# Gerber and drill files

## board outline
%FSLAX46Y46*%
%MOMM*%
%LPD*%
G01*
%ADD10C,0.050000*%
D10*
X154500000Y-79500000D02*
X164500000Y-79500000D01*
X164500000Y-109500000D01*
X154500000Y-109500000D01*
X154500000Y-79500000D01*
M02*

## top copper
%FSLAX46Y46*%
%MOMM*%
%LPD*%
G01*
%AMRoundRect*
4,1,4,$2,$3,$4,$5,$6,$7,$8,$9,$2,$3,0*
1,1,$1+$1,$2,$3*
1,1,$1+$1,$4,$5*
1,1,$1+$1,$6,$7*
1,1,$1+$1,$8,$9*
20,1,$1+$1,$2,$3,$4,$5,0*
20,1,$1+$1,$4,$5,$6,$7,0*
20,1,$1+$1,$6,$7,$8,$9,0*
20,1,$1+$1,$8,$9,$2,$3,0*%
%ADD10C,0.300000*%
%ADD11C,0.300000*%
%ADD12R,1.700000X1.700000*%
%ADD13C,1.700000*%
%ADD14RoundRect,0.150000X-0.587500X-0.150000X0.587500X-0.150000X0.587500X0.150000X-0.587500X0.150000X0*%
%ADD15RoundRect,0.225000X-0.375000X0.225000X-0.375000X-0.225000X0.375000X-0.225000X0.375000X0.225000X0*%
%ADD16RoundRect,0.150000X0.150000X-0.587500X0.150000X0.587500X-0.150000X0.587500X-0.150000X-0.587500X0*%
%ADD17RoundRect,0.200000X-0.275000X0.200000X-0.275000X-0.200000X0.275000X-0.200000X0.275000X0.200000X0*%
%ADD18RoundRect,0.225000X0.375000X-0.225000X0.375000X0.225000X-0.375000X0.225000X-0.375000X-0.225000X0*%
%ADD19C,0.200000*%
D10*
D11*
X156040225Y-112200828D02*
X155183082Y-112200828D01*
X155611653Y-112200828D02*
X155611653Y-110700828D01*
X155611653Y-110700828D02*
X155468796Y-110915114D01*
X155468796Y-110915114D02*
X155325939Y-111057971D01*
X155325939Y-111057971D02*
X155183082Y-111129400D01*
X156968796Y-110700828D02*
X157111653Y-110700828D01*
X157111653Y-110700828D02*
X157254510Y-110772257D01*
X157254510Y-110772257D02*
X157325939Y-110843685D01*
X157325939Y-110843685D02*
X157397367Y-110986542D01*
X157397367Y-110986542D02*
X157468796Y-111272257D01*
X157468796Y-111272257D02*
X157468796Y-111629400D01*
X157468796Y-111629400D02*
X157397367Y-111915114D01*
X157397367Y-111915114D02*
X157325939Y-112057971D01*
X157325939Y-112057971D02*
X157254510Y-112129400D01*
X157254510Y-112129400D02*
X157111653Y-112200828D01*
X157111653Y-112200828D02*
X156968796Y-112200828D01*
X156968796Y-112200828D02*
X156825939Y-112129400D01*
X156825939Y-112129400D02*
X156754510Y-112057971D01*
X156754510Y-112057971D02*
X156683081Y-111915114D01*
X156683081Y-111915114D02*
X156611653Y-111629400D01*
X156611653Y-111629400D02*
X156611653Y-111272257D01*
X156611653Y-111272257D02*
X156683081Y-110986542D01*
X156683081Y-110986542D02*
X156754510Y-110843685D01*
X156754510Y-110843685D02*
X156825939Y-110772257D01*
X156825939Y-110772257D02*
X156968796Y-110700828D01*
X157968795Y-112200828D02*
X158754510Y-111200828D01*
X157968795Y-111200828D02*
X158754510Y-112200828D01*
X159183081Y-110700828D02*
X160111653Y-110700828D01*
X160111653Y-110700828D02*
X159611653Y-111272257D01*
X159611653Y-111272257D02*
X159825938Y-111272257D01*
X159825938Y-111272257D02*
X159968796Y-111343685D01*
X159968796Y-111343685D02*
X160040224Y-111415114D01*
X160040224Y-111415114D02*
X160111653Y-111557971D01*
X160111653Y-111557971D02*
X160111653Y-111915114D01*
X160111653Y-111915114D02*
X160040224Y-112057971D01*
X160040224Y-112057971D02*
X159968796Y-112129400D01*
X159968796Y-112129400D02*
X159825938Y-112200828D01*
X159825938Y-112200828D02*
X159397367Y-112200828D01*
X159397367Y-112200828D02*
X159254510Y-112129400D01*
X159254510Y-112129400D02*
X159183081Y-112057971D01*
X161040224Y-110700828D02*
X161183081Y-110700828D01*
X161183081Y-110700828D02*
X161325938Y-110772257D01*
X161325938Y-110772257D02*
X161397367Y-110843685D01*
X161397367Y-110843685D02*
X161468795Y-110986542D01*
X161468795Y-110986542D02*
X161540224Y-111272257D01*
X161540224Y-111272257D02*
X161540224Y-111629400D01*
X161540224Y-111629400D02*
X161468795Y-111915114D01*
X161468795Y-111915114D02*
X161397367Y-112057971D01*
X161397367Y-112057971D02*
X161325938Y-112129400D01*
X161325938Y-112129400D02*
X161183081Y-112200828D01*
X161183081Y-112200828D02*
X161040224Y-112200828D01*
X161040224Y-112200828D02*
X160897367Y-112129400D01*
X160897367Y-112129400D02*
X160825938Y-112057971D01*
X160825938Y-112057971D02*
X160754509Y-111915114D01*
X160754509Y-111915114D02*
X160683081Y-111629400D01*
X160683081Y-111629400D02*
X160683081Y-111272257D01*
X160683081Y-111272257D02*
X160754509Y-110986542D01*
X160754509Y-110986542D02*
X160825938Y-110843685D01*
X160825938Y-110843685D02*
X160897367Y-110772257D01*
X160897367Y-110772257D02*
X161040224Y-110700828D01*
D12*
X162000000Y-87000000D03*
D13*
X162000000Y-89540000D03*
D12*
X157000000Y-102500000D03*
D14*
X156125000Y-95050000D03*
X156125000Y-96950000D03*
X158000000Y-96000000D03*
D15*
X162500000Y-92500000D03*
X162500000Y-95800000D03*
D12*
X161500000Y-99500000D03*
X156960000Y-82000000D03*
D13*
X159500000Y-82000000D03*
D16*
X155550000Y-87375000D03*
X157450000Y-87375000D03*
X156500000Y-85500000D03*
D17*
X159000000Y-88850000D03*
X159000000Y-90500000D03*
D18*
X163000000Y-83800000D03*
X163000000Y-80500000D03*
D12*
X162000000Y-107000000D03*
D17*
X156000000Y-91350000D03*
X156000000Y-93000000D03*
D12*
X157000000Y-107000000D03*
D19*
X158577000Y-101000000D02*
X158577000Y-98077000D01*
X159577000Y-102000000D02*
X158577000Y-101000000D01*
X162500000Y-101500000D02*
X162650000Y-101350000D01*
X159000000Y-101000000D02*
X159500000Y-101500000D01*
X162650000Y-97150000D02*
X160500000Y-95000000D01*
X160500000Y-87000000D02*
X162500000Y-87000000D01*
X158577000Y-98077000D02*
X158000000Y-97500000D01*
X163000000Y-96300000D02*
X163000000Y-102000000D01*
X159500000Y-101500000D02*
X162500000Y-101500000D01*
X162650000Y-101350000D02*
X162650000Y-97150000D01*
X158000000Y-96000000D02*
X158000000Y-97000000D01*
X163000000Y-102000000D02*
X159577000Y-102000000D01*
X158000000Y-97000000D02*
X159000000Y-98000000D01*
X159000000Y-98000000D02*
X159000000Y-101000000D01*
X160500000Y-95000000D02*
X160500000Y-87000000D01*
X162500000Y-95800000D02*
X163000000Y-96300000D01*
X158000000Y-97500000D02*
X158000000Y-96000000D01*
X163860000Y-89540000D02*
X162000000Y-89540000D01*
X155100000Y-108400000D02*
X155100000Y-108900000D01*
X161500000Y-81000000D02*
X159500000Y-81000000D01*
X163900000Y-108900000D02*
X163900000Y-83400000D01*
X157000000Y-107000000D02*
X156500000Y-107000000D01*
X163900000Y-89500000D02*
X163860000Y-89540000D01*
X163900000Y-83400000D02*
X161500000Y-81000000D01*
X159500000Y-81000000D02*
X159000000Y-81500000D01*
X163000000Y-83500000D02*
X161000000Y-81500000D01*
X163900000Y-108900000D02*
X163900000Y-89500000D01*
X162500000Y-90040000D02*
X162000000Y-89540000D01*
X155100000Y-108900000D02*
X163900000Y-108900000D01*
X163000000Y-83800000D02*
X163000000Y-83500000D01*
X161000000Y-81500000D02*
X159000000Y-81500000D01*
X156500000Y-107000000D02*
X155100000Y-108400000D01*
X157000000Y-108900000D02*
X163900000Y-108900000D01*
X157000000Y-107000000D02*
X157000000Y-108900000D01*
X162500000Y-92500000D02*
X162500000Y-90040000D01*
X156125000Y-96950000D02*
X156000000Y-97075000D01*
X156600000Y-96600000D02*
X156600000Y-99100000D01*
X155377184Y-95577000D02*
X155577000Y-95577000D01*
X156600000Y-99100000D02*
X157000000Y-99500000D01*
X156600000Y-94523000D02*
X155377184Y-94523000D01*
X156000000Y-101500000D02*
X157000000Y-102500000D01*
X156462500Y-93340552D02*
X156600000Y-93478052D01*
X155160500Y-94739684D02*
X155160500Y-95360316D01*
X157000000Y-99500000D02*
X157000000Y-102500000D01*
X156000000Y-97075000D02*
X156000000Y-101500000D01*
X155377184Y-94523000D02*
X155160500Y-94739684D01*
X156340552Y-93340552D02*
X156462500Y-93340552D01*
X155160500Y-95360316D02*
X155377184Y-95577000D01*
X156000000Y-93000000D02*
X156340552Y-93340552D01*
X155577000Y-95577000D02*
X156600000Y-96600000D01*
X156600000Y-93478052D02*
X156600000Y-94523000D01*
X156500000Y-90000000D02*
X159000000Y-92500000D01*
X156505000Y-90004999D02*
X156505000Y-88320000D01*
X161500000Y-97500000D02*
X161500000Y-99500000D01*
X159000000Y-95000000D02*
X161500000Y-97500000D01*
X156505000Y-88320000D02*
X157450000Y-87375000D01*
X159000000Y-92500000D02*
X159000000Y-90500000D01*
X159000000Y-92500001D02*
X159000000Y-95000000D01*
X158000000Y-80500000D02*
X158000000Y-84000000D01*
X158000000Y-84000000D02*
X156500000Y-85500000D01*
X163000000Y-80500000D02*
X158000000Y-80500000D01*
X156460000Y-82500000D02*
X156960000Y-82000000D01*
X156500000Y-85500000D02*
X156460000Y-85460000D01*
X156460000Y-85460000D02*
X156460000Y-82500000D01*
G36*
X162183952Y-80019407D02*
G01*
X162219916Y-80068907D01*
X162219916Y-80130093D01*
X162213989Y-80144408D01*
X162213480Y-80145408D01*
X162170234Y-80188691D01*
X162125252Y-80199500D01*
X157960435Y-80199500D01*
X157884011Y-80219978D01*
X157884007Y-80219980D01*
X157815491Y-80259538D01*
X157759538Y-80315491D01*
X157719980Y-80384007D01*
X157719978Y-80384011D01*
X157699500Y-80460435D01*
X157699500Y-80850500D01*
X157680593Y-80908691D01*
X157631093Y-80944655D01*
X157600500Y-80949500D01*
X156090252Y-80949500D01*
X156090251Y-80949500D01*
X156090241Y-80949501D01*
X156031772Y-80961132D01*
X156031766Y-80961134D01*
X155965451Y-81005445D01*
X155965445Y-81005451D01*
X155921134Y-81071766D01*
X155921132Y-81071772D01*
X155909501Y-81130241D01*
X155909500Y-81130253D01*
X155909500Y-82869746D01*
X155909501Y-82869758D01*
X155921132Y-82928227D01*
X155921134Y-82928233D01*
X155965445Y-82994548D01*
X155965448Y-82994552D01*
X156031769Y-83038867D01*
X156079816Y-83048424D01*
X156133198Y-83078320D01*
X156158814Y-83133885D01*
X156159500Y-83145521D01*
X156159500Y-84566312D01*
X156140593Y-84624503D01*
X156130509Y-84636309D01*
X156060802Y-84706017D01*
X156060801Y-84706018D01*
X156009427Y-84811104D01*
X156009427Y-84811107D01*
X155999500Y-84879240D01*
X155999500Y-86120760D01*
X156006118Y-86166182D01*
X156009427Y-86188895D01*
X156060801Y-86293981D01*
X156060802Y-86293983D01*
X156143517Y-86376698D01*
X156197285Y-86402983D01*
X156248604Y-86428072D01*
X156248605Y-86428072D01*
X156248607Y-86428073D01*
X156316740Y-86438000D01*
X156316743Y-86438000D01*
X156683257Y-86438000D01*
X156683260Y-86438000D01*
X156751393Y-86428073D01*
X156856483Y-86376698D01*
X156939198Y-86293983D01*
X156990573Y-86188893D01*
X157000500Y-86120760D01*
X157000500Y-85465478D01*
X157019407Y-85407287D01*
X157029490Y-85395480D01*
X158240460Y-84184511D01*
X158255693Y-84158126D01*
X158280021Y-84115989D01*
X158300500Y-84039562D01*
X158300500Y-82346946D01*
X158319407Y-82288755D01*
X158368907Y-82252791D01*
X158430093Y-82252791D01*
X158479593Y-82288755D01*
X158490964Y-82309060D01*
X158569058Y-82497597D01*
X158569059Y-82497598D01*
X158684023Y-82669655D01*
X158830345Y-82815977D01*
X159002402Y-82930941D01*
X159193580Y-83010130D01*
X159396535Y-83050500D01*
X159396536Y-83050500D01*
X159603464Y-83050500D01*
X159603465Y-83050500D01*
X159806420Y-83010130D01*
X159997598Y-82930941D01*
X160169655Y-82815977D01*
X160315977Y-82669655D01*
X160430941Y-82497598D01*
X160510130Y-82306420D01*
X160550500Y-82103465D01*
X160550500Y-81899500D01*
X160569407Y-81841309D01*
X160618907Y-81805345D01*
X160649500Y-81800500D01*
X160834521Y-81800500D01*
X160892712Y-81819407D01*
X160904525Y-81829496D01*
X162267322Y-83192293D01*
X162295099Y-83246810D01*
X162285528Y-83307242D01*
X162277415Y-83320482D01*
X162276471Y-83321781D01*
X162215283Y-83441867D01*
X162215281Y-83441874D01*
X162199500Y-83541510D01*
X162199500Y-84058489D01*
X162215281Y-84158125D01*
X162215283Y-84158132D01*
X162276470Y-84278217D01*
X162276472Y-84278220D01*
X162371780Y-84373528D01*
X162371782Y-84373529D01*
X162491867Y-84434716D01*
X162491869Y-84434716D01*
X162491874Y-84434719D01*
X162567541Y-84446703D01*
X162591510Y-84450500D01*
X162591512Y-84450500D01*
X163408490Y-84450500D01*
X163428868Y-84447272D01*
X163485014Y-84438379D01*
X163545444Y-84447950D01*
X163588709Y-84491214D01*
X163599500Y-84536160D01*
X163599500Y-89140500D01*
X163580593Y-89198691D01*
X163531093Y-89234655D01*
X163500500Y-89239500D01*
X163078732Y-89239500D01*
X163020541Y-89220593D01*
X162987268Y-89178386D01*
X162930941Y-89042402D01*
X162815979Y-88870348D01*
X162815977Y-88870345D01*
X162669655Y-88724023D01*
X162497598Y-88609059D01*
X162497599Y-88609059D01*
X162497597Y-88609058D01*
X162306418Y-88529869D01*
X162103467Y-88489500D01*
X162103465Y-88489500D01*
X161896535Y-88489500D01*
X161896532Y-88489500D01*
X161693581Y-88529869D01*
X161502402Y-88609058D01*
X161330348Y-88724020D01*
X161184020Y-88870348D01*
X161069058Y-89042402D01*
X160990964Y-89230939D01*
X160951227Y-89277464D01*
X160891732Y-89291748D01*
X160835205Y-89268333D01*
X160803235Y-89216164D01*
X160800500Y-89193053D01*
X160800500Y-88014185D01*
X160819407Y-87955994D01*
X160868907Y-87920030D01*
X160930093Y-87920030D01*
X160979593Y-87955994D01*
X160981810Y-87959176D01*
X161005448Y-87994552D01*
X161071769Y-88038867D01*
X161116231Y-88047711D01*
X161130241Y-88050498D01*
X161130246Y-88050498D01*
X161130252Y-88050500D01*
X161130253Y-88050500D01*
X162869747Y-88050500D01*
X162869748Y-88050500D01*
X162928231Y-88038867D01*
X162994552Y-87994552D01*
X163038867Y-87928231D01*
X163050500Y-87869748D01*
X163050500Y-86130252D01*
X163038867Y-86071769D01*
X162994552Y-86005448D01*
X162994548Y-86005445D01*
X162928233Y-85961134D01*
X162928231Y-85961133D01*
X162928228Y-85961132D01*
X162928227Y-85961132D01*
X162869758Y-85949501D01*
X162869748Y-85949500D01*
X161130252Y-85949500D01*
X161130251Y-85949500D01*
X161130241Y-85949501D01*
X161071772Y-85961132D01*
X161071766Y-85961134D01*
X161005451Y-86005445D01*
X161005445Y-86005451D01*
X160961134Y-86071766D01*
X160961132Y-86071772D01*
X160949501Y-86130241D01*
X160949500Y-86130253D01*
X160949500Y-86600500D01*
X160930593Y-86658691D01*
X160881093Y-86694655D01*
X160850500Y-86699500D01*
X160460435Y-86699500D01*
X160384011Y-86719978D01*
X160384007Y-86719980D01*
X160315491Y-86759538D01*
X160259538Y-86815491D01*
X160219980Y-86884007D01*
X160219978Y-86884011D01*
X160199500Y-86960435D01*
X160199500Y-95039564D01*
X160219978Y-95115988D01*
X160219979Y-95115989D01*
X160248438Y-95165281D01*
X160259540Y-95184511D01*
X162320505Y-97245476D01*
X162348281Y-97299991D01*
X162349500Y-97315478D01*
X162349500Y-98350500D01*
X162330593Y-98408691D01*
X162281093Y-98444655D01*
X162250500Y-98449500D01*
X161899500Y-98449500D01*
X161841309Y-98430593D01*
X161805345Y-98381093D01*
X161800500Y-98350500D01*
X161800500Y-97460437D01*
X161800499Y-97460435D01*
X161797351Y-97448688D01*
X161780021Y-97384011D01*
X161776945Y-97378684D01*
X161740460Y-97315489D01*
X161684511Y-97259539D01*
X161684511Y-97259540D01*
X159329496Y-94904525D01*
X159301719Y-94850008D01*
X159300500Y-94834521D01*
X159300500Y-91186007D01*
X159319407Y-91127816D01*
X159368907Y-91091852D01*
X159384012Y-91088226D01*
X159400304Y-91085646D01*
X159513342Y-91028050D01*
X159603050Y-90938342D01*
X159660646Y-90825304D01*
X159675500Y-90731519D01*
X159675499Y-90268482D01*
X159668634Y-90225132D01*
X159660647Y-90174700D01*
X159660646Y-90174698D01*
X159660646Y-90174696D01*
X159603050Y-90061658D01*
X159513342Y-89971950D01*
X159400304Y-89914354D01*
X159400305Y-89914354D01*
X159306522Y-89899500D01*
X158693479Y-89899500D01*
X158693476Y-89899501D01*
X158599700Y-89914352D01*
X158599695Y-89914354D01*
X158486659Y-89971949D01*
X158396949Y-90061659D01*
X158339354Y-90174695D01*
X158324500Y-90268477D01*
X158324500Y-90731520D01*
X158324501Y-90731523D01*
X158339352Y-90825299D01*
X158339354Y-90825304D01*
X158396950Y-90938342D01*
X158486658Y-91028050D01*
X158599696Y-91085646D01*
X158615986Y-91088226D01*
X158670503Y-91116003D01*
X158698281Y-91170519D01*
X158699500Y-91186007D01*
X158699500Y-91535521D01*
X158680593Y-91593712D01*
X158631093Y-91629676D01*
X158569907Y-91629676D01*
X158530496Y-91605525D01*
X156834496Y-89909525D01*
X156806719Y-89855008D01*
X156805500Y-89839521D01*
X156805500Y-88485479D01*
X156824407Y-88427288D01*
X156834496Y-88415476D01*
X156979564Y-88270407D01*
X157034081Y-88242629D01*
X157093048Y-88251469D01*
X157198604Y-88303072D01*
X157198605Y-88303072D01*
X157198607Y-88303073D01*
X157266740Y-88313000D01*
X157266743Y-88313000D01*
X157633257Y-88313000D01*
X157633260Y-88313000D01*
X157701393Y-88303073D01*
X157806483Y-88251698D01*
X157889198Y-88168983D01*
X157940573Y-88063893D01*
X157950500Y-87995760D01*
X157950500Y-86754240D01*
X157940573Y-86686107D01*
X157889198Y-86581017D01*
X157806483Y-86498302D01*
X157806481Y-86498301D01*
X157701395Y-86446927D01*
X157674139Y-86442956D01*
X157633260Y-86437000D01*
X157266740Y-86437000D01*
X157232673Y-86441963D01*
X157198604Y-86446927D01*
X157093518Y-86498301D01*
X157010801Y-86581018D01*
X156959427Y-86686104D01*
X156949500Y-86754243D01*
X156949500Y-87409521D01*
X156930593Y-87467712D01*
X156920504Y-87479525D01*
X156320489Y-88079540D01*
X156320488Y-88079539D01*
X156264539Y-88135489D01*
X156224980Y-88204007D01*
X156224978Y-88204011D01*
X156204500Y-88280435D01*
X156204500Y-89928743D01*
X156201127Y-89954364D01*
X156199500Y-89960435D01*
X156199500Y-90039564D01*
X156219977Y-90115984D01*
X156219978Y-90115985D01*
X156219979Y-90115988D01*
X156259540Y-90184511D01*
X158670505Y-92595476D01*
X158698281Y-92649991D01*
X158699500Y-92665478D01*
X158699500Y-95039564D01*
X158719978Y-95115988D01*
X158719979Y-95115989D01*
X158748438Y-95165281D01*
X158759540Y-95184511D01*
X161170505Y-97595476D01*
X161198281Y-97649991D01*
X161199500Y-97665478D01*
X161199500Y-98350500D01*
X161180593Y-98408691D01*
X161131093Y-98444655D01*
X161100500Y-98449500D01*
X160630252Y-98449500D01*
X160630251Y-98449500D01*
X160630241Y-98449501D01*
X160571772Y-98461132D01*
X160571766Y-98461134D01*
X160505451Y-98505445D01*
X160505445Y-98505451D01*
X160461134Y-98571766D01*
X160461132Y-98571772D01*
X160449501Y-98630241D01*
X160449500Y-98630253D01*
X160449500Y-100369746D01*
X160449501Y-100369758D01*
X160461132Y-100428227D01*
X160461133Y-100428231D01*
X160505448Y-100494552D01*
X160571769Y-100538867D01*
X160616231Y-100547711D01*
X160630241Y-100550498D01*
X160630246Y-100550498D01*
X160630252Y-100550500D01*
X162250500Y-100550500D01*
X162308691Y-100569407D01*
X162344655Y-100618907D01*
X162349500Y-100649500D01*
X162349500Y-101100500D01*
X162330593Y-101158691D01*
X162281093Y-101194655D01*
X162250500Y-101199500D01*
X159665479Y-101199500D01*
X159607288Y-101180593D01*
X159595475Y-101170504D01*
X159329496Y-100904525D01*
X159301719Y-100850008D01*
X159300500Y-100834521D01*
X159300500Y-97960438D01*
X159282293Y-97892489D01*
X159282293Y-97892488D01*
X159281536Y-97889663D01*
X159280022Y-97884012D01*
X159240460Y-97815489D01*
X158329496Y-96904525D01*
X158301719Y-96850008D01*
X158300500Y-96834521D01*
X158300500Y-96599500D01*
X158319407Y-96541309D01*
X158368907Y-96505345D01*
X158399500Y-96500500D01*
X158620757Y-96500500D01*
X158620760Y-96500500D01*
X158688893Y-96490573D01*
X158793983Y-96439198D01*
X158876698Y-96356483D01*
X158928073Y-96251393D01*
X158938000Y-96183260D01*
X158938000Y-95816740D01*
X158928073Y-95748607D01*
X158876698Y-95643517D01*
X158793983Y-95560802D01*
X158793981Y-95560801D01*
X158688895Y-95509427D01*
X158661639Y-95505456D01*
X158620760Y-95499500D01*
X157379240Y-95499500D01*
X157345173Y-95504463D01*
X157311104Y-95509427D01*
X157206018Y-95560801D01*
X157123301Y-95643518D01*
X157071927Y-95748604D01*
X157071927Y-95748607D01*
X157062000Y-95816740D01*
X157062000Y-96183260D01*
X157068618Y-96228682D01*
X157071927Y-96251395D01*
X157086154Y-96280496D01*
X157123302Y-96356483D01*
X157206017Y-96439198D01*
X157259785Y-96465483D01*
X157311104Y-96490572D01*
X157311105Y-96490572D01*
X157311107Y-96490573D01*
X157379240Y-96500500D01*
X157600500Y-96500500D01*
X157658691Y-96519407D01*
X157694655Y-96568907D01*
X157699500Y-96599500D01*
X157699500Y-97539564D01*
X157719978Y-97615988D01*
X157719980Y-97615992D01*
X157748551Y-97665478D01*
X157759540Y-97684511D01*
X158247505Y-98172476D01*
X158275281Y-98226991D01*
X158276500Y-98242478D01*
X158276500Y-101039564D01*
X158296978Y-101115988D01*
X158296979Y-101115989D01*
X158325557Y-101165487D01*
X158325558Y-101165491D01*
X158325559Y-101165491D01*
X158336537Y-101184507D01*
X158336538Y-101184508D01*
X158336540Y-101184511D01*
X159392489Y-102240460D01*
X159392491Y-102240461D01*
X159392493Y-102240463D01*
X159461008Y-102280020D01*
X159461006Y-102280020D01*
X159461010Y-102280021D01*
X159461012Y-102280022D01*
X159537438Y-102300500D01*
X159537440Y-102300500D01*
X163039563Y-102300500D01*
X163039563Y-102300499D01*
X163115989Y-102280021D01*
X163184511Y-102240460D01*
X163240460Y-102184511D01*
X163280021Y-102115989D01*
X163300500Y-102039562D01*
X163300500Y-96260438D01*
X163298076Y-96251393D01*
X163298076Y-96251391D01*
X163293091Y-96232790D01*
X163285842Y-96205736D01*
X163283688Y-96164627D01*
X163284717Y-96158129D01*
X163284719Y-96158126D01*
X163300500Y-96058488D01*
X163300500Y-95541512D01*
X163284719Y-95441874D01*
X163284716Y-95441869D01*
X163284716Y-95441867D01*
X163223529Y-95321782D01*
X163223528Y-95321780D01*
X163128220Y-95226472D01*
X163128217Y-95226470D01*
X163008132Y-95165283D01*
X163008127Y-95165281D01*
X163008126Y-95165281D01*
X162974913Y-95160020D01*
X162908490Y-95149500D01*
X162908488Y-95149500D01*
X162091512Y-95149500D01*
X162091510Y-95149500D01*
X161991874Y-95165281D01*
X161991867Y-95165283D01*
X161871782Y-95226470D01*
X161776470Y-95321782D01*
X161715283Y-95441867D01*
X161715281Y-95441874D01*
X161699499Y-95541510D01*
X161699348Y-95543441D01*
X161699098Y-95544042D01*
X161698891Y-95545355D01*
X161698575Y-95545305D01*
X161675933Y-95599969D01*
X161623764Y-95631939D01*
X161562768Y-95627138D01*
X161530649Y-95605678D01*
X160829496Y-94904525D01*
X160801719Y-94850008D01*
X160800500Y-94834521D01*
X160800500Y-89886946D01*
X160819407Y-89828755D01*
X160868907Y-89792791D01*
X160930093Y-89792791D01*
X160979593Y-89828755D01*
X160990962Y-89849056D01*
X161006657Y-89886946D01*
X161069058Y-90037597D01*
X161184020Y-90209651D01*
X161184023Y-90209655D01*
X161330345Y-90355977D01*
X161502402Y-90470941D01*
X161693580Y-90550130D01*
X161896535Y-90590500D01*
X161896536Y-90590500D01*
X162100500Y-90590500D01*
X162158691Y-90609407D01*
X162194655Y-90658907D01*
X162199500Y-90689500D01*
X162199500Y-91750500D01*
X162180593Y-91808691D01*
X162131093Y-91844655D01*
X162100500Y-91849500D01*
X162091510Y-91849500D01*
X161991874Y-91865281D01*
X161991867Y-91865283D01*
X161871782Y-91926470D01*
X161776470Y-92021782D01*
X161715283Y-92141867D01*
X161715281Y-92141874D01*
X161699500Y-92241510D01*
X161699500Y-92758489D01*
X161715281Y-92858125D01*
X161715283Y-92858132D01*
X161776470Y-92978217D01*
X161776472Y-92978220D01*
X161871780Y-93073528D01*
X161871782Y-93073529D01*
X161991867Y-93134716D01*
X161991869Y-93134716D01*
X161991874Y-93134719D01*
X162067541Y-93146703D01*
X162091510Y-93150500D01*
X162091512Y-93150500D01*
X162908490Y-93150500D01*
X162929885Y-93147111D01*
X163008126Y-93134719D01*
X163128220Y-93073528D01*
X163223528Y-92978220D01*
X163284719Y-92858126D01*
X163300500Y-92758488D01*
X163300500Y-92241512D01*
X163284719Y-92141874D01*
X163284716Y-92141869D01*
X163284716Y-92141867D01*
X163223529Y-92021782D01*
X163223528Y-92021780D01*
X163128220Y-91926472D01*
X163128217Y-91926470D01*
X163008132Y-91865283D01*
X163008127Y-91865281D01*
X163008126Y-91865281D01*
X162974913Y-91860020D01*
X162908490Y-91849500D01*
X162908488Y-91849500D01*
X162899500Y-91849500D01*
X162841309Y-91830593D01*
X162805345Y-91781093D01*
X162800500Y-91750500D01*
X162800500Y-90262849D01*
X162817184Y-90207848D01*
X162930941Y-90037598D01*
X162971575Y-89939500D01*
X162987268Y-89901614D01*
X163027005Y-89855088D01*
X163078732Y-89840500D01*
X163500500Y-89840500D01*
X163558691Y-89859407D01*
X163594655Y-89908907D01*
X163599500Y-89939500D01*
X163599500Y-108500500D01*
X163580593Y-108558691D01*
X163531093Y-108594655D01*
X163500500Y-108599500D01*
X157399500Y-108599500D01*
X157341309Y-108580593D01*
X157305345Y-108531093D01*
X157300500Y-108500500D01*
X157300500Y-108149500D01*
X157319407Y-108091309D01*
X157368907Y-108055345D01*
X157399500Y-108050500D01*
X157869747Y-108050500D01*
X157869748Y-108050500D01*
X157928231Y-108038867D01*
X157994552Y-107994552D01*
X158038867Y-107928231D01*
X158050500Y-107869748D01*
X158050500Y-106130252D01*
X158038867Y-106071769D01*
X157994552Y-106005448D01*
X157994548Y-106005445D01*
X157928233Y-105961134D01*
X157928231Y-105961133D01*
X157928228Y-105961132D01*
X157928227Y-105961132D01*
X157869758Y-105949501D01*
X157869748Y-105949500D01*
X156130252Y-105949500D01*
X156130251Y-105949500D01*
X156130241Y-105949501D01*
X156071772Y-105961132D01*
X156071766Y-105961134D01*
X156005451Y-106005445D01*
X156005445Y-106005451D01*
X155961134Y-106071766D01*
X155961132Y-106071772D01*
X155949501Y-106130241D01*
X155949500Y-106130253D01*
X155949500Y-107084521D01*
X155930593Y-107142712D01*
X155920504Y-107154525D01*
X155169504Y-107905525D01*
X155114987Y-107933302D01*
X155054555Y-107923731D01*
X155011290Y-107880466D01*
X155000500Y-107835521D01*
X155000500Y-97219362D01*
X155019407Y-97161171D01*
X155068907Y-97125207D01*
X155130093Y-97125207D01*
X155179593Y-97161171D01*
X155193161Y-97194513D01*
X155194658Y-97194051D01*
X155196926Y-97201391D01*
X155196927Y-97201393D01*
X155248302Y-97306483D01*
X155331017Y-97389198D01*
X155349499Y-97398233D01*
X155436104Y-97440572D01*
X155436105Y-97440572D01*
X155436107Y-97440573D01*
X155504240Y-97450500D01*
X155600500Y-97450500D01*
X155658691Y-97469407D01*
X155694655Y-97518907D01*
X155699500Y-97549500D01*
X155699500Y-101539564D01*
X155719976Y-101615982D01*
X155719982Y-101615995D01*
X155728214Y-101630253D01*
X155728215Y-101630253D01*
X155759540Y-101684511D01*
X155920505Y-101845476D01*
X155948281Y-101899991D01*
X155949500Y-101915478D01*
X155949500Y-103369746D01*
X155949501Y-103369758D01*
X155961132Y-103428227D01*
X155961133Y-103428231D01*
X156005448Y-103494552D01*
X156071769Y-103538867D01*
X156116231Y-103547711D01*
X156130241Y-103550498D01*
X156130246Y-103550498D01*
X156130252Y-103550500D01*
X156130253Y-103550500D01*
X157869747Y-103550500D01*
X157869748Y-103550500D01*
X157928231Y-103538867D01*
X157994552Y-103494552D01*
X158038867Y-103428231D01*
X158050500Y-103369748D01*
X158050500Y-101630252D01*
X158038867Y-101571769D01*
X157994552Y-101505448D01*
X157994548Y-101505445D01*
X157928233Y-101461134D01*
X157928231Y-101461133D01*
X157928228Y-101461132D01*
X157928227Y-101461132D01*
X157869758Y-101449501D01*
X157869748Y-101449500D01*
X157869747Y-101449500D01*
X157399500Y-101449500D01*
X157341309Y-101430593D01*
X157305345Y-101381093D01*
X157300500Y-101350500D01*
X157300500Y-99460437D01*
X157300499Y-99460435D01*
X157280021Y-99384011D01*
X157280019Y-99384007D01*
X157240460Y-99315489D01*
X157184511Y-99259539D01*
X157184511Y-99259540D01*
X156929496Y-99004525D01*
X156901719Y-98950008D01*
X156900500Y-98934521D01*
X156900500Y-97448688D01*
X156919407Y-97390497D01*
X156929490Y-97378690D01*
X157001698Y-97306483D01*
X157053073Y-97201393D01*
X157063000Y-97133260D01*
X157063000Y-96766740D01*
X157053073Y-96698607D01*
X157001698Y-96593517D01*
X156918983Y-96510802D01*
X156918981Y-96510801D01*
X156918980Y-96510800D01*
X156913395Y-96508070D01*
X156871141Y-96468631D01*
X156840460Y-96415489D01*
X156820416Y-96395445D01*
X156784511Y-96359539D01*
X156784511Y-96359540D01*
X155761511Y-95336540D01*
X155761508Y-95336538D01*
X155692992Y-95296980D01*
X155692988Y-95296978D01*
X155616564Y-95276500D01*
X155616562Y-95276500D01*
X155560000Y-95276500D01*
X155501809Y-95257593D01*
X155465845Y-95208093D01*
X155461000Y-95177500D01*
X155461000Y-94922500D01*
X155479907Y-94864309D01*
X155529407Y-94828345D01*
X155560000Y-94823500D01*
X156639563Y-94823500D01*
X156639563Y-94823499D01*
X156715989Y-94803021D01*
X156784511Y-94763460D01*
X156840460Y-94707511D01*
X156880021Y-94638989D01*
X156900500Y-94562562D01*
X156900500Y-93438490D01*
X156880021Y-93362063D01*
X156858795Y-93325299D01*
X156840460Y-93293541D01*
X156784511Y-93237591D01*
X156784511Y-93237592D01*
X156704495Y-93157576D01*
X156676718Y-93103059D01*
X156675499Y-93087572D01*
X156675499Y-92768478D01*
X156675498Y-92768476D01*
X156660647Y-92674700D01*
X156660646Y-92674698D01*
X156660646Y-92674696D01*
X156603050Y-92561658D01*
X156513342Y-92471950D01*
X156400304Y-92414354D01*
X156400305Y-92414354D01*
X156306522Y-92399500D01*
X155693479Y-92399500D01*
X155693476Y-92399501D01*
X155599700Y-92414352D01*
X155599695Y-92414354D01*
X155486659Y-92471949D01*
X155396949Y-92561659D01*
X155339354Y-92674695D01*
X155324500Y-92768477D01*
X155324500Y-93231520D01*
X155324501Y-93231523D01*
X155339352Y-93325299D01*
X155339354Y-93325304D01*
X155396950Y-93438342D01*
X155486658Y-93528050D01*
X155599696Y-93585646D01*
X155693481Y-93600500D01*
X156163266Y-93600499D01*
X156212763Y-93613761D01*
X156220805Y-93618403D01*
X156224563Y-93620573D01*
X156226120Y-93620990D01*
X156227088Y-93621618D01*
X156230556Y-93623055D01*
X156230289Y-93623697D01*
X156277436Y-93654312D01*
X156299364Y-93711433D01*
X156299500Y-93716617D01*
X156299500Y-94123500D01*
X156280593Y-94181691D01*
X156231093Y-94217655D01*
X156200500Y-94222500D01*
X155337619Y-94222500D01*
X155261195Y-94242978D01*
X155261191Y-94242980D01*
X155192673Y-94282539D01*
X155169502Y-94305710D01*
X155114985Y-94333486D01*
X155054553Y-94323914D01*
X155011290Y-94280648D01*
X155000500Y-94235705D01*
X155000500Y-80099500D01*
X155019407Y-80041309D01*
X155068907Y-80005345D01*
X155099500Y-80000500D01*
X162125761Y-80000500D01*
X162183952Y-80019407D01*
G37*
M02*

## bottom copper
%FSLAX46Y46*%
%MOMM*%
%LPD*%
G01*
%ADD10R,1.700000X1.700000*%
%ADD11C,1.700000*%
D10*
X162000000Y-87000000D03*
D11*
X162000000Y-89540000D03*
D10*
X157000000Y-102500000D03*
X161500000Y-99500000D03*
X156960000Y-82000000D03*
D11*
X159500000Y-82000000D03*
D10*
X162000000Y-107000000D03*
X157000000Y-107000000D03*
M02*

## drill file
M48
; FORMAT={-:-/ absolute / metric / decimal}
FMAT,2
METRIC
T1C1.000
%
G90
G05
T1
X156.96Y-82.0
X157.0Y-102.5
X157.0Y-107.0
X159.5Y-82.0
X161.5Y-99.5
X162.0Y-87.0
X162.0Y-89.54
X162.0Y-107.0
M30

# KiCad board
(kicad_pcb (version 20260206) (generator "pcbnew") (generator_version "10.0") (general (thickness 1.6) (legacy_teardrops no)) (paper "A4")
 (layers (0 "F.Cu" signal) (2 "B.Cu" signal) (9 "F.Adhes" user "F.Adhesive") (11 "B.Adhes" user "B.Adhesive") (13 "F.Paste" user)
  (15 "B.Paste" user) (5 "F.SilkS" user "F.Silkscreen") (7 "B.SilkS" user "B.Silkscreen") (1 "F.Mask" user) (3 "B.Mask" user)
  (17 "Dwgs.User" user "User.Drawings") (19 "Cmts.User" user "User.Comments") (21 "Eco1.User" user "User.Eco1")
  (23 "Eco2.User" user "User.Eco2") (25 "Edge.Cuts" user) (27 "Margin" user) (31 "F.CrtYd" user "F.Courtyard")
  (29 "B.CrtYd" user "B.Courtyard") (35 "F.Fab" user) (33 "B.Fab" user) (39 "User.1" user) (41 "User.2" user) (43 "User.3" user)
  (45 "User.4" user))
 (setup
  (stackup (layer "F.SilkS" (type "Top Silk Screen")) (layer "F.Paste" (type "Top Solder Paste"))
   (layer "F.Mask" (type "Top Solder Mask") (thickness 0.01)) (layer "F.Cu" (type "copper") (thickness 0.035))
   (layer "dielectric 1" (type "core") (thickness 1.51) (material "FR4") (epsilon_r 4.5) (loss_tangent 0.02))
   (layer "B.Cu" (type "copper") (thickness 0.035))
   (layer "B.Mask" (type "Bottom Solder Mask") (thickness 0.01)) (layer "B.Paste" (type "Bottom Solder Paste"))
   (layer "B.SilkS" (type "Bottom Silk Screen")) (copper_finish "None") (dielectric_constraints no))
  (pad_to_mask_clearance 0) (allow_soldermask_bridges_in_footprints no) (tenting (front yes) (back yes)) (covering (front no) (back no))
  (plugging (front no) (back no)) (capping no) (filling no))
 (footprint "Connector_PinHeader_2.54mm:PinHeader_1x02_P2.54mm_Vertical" (layer "F.Cu") (at 162 87)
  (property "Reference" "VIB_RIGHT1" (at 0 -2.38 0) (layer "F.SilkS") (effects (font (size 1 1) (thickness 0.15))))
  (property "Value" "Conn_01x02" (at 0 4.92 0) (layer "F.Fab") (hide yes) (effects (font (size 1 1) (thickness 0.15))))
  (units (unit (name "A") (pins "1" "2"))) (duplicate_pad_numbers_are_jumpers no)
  (pad "1" thru_hole rect (at 0 0) (size 1.7 1.7) (drill 1) (layers "*.Cu" "*.Mask") (remove_unused_layers no) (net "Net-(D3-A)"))
  (pad "2" thru_hole circle (at 0 2.54) (size 1.7 1.7) (drill 1) (layers "*.Cu" "*.Mask") (remove_unused_layers no) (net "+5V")))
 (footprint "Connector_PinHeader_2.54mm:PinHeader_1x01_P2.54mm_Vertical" (layer "F.Cu") (at 157 102.5)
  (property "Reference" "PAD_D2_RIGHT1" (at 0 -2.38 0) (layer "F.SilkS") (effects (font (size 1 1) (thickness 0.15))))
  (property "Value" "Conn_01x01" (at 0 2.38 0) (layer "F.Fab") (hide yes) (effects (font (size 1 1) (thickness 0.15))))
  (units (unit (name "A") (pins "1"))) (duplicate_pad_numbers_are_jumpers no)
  (pad "1" thru_hole rect (at 0 0) (size 1.7 1.7) (drill 1) (layers "*.Cu" "*.Mask") (remove_unused_layers no)
   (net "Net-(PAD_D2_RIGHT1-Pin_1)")))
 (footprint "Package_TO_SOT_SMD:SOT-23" (layer "F.Cu") (at 157.0625 96)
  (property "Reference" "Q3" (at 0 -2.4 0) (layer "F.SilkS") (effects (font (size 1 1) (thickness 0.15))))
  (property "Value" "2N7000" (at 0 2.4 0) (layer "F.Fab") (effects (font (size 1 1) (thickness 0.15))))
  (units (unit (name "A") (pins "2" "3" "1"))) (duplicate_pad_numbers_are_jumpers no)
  (pad "1" smd roundrect (at -0.9375 -0.95) (size 1.475 0.6) (layers "F.Cu" "F.Mask" "F.Paste") (roundrect_rratio 0.25) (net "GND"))
  (pad "2" smd roundrect (at -0.9375 0.95) (size 1.475 0.6) (layers "F.Cu" "F.Mask" "F.Paste") (roundrect_rratio 0.25)
   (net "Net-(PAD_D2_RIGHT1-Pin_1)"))
  (pad "3" smd roundrect (at 0.9375 0) (size 1.475 0.6) (layers "F.Cu" "F.Mask" "F.Paste") (roundrect_rratio 0.25) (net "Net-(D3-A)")))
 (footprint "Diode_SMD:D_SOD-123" (layer "F.Cu") (at 162.5 94.15 -90)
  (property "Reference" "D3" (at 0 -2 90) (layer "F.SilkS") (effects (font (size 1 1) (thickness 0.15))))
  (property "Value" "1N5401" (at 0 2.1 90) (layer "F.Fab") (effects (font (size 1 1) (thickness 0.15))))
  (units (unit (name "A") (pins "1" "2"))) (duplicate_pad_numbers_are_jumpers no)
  (pad "1" smd roundrect (at -1.65 0 270) (size 0.9 1.2) (layers "F.Cu" "F.Mask" "F.Paste") (roundrect_rratio 0.25) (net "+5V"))
  (pad "2" smd roundrect (at 1.65 0 270) (size 0.9 1.2) (layers "F.Cu" "F.Mask" "F.Paste") (roundrect_rratio 0.25) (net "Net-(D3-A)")))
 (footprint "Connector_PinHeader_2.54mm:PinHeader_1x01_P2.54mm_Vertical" (layer "F.Cu") (at 161.5 99.5)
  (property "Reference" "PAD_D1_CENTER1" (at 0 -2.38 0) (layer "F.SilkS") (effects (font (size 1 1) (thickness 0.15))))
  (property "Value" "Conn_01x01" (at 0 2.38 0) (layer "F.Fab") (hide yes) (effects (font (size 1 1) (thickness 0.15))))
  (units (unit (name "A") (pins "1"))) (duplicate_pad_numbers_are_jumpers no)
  (pad "1" thru_hole rect (at 0 0) (size 1.7 1.7) (drill 1) (layers "*.Cu" "*.Mask") (remove_unused_layers no)
   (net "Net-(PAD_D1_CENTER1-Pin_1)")))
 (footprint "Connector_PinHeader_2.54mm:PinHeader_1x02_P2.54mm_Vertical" (layer "F.Cu") (at 156.96 82 90)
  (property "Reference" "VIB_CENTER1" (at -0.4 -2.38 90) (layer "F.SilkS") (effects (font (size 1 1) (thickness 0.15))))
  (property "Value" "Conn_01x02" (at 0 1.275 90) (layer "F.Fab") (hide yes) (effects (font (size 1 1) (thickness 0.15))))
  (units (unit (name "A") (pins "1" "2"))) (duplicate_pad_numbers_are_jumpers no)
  (pad "1" thru_hole rect (at 0 0 90) (size 1.7 1.7) (drill 1) (layers "*.Cu" "*.Mask") (remove_unused_layers no) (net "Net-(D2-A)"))
  (pad "2" thru_hole circle (at 0 2.54 90) (size 1.7 1.7) (drill 1) (layers "*.Cu" "*.Mask") (remove_unused_layers no) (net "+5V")))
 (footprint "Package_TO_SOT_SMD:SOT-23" (layer "F.Cu") (at 156.5 86.4375 90)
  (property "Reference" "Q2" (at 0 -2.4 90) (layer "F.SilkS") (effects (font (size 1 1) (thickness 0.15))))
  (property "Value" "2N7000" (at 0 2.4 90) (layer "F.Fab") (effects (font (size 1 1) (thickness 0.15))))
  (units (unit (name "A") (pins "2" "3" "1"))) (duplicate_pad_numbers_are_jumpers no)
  (pad "1" smd roundrect (at -0.9375 -0.95 90) (size 1.475 0.6) (layers "F.Cu" "F.Mask" "F.Paste") (roundrect_rratio 0.25) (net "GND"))
  (pad "2" smd roundrect (at -0.9375 0.95 90) (size 1.475 0.6) (layers "F.Cu" "F.Mask" "F.Paste") (roundrect_rratio 0.25)
   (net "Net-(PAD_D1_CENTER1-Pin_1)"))
  (pad "3" smd roundrect (at 0.9375 0 90) (size 1.475 0.6) (layers "F.Cu" "F.Mask" "F.Paste") (roundrect_rratio 0.25) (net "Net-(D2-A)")))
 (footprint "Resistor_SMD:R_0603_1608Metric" (layer "F.Cu") (at 159 89.675 -90)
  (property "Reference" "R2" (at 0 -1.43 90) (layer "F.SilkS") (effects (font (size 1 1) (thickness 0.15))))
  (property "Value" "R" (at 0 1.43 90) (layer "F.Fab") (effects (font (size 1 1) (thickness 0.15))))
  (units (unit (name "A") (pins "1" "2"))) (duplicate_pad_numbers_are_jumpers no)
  (pad "1" smd roundrect (at -0.825 0 270) (size 0.8 0.95) (layers "F.Cu" "F.Mask" "F.Paste") (roundrect_rratio 0.25) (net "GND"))
  (pad "2" smd roundrect (at 0.825 0 270) (size 0.8 0.95) (layers "F.Cu" "F.Mask" "F.Paste") (roundrect_rratio 0.25)
   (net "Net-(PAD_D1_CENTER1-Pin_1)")))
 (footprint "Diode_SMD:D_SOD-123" (layer "F.Cu") (at 163 82.15 90)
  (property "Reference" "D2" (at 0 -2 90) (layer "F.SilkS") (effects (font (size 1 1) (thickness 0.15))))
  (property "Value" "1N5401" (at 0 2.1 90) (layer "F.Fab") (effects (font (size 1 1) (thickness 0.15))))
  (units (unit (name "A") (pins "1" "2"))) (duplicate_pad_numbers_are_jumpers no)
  (pad "1" smd roundrect (at -1.65 0 90) (size 0.9 1.2) (layers "F.Cu" "F.Mask" "F.Paste") (roundrect_rratio 0.25) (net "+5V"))
  (pad "2" smd roundrect (at 1.65 0 90) (size 0.9 1.2) (layers "F.Cu" "F.Mask" "F.Paste") (roundrect_rratio 0.25) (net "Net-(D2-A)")))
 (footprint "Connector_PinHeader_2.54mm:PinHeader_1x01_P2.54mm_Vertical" (layer "F.Cu") (at 162 107)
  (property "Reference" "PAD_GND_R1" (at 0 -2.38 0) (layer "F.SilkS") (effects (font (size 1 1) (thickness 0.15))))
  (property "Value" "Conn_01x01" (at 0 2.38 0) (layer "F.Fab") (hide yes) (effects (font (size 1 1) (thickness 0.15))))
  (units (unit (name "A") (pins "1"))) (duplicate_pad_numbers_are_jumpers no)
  (pad "1" thru_hole rect (at 0 0) (size 1.7 1.7) (drill 1) (layers "*.Cu" "*.Mask") (remove_unused_layers no) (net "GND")))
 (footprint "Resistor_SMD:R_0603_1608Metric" (layer "F.Cu") (at 156 92.175 -90)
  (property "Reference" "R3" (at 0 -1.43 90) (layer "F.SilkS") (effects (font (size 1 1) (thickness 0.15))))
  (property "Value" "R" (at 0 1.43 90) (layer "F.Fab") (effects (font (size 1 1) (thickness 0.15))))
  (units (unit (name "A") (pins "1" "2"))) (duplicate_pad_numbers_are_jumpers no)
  (pad "1" smd roundrect (at -0.825 0 270) (size 0.8 0.95) (layers "F.Cu" "F.Mask" "F.Paste") (roundrect_rratio 0.25) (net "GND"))
  (pad "2" smd roundrect (at 0.825 0 270) (size 0.8 0.95) (layers "F.Cu" "F.Mask" "F.Paste") (roundrect_rratio 0.25)
   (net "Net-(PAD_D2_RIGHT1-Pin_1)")))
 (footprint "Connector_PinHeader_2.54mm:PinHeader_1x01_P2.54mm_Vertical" (layer "F.Cu") (at 157 107)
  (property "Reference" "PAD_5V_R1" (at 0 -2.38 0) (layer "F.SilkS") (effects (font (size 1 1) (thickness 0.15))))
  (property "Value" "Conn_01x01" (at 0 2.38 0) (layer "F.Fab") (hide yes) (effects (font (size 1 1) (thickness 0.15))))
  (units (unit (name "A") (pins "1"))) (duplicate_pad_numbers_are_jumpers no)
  (pad "1" thru_hole rect (at 0 0) (size 1.7 1.7) (drill 1) (layers "*.Cu" "*.Mask") (remove_unused_layers no) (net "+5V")))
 (gr_rect (start 154.5 79.5) (end 164.5 109.5) (stroke (width 0.05) (type default)) (fill no) (layer "Edge.Cuts"))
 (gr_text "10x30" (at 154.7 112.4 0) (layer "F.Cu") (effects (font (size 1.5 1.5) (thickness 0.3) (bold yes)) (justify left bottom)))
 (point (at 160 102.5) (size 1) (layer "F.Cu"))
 (segment (start 158.577 101) (end 158.577 98.077) (width 0.2) (layer "F.Cu") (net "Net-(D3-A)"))
 (segment (start 159.577 102) (end 158.577 101) (width 0.2) (layer "F.Cu") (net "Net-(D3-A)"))
 (segment (start 162.5 101.5) (end 162.65 101.35) (width 0.2) (layer "F.Cu") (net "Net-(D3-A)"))
 (segment (start 159 101) (end 159.5 101.5) (width 0.2) (layer "F.Cu") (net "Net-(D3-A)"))
 (segment (start 162.65 97.15) (end 160.5 95) (width 0.2) (layer "F.Cu") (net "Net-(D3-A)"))
 (segment (start 160.5 87) (end 162.5 87) (width 0.2) (layer "F.Cu") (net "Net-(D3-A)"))
 (segment (start 158.577 98.077) (end 158 97.5) (width 0.2) (layer "F.Cu") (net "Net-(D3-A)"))
 (segment (start 163 96.3) (end 163 102) (width 0.2) (layer "F.Cu") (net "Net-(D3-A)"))
 (segment (start 159.5 101.5) (end 162.5 101.5) (width 0.2) (layer "F.Cu") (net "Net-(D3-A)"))
 (segment (start 162.65 101.35) (end 162.65 97.15) (width 0.2) (layer "F.Cu") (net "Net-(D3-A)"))
 (segment (start 158 96) (end 158 97) (width 0.2) (layer "F.Cu") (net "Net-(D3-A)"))
 (segment (start 163 102) (end 159.577 102) (width 0.2) (layer "F.Cu") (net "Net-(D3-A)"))
 (segment (start 158 97) (end 159 98) (width 0.2) (layer "F.Cu") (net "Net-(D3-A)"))
 (segment (start 159 98) (end 159 101) (width 0.2) (layer "F.Cu") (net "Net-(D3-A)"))
 (segment (start 160.5 95) (end 160.5 87) (width 0.2) (layer "F.Cu") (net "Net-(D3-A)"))
 (segment (start 162.5 95.8) (end 163 96.3) (width 0.2) (layer "F.Cu") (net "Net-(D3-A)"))
 (segment (start 158 97.5) (end 158 96) (width 0.2) (layer "F.Cu") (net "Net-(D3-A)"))
 (segment (start 163.86 89.54) (end 162 89.54) (width 0.2) (layer "F.Cu") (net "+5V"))
 (segment (start 155.1 108.4) (end 155.1 108.9) (width 0.2) (layer "F.Cu") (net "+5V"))
 (segment (start 161.5 81) (end 159.5 81) (width 0.2) (layer "F.Cu") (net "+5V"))
 (segment (start 163.9 108.9) (end 163.9 83.4) (width 0.2) (layer "F.Cu") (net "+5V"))
 (segment (start 157 107) (end 156.5 107) (width 0.2) (layer "F.Cu") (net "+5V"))
 (segment (start 163.9 89.5) (end 163.86 89.54) (width 0.2) (layer "F.Cu") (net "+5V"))
 (segment (start 163.9 83.4) (end 161.5 81) (width 0.2) (layer "F.Cu") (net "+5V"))
 (segment (start 159.5 81) (end 159 81.5) (width 0.2) (layer "F.Cu") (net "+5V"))
 (segment (start 163 83.5) (end 161 81.5) (width 0.2) (layer "F.Cu") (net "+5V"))
 (segment (start 163.9 108.9) (end 163.9 89.5) (width 0.2) (layer "F.Cu") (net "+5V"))
 (segment (start 162.5 90.04) (end 162 89.54) (width 0.2) (layer "F.Cu") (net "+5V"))
 (segment (start 155.1 108.9) (end 163.9 108.9) (width 0.2) (layer "F.Cu") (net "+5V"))
 (segment (start 163 83.8) (end 163 83.5) (width 0.2) (layer "F.Cu") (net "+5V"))
 (segment (start 161 81.5) (end 159 81.5) (width 0.2) (layer "F.Cu") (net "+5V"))
 (segment (start 156.5 107) (end 155.1 108.4) (width 0.2) (layer "F.Cu") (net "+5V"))
 (segment (start 157 108.9) (end 163.9 108.9) (width 0.2) (layer "F.Cu") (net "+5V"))
 (segment (start 157 107) (end 157 108.9) (width 0.2) (layer "F.Cu") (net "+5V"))
 (segment (start 162.5 92.5) (end 162.5 90.04) (width 0.2) (layer "F.Cu") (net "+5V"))
 (segment (start 156.125 96.95) (end 156 97.075) (width 0.2) (layer "F.Cu") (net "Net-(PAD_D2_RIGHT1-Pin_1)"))
 (segment (start 156.6 96.6) (end 156.6 99.1) (width 0.2) (layer "F.Cu") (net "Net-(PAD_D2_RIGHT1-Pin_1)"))
 (segment (start 155.377184 95.577) (end 155.577 95.577) (width 0.2) (layer "F.Cu") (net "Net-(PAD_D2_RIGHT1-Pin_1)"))
 (segment (start 156.6 99.1) (end 157 99.5) (width 0.2) (layer "F.Cu") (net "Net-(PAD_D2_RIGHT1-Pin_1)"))
 (segment (start 156.6 94.523) (end 155.377184 94.523) (width 0.2) (layer "F.Cu") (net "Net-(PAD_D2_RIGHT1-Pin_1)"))
 (segment (start 156 101.5) (end 157 102.5) (width 0.2) (layer "F.Cu") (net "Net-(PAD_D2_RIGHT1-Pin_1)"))
 (segment (start 156.4625 93.340552) (end 156.6 93.478052) (width 0.2) (layer "F.Cu") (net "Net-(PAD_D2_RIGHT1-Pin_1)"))
 (segment (start 155.1605 94.739684) (end 155.1605 95.360316) (width 0.2) (layer "F.Cu") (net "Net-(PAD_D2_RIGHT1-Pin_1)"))
 (segment (start 157 99.5) (end 157 102.5) (width 0.2) (layer "F.Cu") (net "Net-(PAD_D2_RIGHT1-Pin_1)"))
 (segment (start 156 97.075) (end 156 101.5) (width 0.2) (layer "F.Cu") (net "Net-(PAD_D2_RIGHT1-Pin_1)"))
 (segment (start 155.377184 94.523) (end 155.1605 94.739684) (width 0.2) (layer "F.Cu") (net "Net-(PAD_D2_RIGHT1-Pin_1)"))
 (segment (start 156.340552 93.340552) (end 156.4625 93.340552) (width 0.2) (layer "F.Cu") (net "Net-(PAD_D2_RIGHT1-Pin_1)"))
 (segment (start 155.1605 95.360316) (end 155.377184 95.577) (width 0.2) (layer "F.Cu") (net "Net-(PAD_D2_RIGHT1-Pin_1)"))
 (segment (start 156 93) (end 156.340552 93.340552) (width 0.2) (layer "F.Cu") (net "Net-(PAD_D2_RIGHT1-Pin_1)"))
 (segment (start 155.577 95.577) (end 156.6 96.6) (width 0.2) (layer "F.Cu") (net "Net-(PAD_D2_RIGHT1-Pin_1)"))
 (segment (start 156.6 93.478052) (end 156.6 94.523) (width 0.2) (layer "F.Cu") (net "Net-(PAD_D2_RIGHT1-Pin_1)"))
 (segment (start 156.5 90) (end 159 92.5) (width 0.2) (layer "F.Cu") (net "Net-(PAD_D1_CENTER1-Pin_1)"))
 (segment (start 156.505 90.004999) (end 156.505 88.32) (width 0.2) (layer "F.Cu") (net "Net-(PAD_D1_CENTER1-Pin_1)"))
 (segment (start 161.5 97.5) (end 161.5 99.5) (width 0.2) (layer "F.Cu") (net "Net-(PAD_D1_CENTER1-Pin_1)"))
 (segment (start 159 95) (end 161.5 97.5) (width 0.2) (layer "F.Cu") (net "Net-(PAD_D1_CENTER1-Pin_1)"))
 (segment (start 156.505 88.32) (end 157.45 87.375) (width 0.2) (layer "F.Cu") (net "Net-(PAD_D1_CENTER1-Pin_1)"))
 (segment (start 159 92.5) (end 159 90.5) (width 0.2) (layer "F.Cu") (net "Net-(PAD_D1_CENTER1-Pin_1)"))
 (segment (start 159 92.500001) (end 159 95) (width 0.2) (layer "F.Cu") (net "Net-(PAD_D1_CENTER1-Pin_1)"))
 (segment (start 158 80.5) (end 158 84) (width 0.2) (layer "F.Cu") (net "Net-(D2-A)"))
 (segment (start 158 84) (end 156.5 85.5) (width 0.2) (layer "F.Cu") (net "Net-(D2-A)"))
 (segment (start 163 80.5) (end 158 80.5) (width 0.2) (layer "F.Cu") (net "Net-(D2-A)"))
 (segment (start 156.46 82.5) (end 156.96 82) (width 0.2) (layer "F.Cu") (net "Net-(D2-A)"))
 (segment (start 156.5 85.5) (end 156.46 85.46) (width 0.2) (layer "F.Cu") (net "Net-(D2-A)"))
 (segment (start 156.46 85.46) (end 156.46 82.5) (width 0.2) (layer "F.Cu") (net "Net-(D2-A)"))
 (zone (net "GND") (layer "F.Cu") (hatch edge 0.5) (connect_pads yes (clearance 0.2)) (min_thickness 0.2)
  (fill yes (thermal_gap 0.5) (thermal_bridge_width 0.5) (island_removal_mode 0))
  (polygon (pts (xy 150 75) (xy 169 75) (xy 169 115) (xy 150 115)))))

